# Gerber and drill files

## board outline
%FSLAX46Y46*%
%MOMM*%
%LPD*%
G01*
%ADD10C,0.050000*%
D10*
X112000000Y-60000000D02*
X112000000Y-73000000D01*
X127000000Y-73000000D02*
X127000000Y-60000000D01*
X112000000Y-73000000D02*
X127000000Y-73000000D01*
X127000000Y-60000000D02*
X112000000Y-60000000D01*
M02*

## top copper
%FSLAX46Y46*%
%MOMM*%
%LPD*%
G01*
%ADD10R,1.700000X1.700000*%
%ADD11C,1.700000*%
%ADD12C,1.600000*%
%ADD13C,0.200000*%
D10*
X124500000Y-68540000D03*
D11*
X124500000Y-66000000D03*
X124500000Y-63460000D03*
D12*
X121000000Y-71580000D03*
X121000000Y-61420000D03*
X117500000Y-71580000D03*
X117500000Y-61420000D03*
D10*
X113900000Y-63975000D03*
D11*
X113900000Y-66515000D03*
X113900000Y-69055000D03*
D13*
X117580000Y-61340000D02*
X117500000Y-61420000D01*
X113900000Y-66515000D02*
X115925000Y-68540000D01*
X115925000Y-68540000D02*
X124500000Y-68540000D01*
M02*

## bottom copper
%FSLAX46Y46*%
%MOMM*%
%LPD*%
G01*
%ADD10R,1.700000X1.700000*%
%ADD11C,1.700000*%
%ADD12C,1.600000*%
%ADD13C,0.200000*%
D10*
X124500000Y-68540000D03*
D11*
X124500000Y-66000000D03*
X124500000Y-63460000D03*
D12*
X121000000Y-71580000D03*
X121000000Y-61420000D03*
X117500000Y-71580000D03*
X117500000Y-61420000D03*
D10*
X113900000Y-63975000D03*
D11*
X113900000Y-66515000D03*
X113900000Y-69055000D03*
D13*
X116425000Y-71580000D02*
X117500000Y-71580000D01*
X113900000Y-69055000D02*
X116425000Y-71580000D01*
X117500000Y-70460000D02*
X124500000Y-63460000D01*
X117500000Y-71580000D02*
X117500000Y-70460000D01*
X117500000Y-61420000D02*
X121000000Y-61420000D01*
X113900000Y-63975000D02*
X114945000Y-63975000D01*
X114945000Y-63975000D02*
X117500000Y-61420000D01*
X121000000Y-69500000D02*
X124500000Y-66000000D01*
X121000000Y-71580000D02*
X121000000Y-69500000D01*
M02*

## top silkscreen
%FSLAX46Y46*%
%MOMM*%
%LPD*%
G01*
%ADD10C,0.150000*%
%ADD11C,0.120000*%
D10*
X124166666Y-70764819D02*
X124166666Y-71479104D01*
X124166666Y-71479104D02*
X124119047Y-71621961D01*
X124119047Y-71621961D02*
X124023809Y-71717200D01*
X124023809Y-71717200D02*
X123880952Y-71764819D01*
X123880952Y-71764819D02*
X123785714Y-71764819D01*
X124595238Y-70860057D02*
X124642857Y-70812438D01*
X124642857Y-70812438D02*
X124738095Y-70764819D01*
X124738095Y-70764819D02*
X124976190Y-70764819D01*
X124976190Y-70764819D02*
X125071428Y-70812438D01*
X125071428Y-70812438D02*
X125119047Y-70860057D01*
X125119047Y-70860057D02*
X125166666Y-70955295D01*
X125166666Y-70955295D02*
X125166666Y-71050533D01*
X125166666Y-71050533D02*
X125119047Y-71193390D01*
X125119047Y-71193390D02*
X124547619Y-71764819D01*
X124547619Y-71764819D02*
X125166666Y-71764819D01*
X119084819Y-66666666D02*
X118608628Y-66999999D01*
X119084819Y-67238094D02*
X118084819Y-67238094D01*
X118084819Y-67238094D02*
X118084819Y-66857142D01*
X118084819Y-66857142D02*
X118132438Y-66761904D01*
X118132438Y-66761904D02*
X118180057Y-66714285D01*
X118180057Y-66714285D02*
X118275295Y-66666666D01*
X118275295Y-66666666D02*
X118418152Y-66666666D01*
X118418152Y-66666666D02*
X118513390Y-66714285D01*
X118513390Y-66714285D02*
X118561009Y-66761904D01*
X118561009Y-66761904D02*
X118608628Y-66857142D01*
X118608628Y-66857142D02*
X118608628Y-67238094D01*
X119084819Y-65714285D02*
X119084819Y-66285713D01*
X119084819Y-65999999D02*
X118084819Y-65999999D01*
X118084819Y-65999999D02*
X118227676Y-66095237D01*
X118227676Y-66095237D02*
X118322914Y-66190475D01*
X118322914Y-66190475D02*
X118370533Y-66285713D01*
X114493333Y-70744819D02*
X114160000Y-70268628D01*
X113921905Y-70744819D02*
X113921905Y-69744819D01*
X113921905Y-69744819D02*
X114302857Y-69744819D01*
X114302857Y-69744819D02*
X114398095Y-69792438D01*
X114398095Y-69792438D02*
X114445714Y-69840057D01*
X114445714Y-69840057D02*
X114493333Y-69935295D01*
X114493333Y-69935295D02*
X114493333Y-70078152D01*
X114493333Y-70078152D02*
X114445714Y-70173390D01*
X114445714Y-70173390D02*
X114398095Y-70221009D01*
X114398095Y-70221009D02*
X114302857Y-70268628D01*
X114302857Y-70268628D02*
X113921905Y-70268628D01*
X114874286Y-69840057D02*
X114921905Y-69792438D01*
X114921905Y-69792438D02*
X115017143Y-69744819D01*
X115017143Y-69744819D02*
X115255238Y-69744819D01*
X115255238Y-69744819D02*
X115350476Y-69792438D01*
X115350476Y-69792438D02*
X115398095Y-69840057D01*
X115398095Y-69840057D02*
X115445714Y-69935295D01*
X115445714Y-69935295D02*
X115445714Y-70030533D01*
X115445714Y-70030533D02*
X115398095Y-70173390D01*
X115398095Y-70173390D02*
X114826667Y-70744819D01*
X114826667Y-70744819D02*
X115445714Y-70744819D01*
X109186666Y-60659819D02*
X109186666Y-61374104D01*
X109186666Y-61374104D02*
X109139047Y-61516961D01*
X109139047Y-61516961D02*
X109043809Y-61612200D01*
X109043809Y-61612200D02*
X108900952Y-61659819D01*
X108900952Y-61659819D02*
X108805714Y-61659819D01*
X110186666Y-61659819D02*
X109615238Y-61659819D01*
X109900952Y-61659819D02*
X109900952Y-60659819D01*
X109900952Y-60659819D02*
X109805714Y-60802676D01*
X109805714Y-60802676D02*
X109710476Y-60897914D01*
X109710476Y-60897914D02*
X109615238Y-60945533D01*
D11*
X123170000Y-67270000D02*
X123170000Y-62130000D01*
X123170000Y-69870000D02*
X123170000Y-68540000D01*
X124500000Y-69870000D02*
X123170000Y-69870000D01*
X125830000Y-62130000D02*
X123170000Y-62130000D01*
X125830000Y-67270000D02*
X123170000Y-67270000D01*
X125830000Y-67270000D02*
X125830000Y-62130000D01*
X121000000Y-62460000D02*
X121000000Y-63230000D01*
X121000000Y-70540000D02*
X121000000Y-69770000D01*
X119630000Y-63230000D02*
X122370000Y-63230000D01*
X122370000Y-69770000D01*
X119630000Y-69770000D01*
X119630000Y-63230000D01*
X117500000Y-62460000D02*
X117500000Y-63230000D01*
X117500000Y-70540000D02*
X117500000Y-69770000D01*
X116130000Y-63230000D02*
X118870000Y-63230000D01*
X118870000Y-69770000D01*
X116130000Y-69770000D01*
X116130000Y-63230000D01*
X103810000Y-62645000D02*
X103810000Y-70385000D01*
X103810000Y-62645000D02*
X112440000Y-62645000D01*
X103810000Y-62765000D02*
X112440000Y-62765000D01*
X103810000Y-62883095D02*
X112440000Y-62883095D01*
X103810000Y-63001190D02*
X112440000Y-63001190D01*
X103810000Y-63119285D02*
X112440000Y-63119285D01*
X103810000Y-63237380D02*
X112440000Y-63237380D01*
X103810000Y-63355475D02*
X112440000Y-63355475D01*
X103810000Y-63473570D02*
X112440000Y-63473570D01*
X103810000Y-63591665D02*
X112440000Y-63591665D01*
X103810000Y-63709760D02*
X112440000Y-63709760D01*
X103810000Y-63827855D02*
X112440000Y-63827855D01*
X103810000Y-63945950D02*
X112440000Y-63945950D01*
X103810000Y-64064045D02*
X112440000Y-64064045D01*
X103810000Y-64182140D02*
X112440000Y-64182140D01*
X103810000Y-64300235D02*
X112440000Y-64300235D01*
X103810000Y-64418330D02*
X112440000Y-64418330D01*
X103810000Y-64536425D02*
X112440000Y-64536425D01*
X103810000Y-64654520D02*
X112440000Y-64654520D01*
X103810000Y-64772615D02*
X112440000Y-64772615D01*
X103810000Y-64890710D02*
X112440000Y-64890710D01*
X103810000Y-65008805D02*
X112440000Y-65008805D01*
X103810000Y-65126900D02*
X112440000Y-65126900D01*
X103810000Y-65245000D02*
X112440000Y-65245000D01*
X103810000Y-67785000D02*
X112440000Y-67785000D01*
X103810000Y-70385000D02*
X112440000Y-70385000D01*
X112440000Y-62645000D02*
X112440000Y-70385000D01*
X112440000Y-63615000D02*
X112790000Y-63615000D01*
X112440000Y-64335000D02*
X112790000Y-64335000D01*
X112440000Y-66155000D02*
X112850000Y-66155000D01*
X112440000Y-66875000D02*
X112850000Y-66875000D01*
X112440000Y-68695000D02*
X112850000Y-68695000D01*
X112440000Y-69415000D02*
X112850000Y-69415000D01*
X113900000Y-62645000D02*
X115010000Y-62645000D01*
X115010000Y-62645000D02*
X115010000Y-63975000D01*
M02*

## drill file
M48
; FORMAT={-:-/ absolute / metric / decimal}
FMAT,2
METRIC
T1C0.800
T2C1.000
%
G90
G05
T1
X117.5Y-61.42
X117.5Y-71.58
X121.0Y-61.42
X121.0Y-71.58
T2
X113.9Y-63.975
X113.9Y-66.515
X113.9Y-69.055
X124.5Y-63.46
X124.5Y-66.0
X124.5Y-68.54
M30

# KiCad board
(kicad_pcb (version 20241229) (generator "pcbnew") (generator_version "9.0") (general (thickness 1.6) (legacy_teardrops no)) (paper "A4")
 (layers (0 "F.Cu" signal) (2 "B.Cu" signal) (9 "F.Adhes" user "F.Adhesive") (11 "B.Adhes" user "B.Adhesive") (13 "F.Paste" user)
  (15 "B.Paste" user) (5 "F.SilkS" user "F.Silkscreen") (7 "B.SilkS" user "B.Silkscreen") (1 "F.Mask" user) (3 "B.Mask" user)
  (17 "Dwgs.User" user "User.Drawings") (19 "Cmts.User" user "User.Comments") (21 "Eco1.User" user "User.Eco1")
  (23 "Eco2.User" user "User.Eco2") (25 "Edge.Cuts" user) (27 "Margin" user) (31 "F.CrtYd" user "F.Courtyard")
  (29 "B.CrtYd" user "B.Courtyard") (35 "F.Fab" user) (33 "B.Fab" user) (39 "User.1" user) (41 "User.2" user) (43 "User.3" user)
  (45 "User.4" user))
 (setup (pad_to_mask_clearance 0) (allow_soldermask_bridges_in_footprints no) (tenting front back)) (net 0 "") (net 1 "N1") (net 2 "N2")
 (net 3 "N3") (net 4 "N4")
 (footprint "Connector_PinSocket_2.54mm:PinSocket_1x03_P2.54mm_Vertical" (layer "F.Cu") (at 124.5 68.54 180)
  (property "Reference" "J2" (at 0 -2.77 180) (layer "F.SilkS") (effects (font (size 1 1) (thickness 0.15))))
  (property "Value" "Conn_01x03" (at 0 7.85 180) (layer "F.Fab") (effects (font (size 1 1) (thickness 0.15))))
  (fp_line (start 1.33 1.27) (end 1.33 6.41) (stroke (width 0.12) (type solid)) (layer "F.SilkS"))
  (fp_line (start 1.33 -1.33) (end 1.33 0) (stroke (width 0.12) (type solid)) (layer "F.SilkS"))
  (fp_line (start 0 -1.33) (end 1.33 -1.33) (stroke (width 0.12) (type solid)) (layer "F.SilkS"))
  (fp_line (start -1.33 6.41) (end 1.33 6.41) (stroke (width 0.12) (type solid)) (layer "F.SilkS"))
  (fp_line (start -1.33 1.27) (end 1.33 1.27) (stroke (width 0.12) (type solid)) (layer "F.SilkS"))
  (fp_line (start -1.33 1.27) (end -1.33 6.41) (stroke (width 0.12) (type solid)) (layer "F.SilkS"))
  (pad "1" thru_hole rect (at 0 0 180) (size 1.7 1.7) (drill 1) (layers "*.Cu" "*.Mask") (remove_unused_layers no) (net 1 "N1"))
  (pad "2" thru_hole circle (at 0 2.54 180) (size 1.7 1.7) (drill 1) (layers "*.Cu" "*.Mask") (remove_unused_layers no) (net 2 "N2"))
  (pad "3" thru_hole circle (at 0 5.08 180) (size 1.7 1.7) (drill 1) (layers "*.Cu" "*.Mask") (remove_unused_layers no) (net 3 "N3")))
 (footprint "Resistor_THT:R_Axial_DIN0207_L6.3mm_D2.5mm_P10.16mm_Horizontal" (layer "F.Cu") (at 121 71.58 90)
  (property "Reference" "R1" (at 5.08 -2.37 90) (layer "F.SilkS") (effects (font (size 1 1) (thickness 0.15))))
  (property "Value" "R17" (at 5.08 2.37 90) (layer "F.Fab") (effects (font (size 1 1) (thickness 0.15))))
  (fp_line (start 9.12 0) (end 8.35 0) (stroke (width 0.12) (type solid)) (layer "F.SilkS"))
  (fp_line (start 1.04 0) (end 1.81 0) (stroke (width 0.12) (type solid)) (layer "F.SilkS"))
  (fp_rect (start 1.81 -1.37) (end 8.35 1.37) (stroke (width 0.12) (type solid)) (fill no) (layer "F.SilkS"))
  (pad "1" thru_hole circle (at 0 0 90) (size 1.6 1.6) (drill 0.8) (layers "*.Cu" "*.Mask") (remove_unused_layers no) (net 2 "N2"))
  (pad "2" thru_hole circle (at 10.16 0 90) (size 1.6 1.6) (drill 0.8) (layers "*.Cu" "*.Mask") (remove_unused_layers no) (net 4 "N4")))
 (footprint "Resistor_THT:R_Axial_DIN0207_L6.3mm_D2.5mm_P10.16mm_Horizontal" (layer "F.Cu") (at 117.5 71.58 90)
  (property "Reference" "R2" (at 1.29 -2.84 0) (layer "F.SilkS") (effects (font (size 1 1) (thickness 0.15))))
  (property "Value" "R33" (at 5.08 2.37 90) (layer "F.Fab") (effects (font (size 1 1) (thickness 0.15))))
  (fp_line (start 9.12 0) (end 8.35 0) (stroke (width 0.12) (type solid)) (layer "F.SilkS"))
  (fp_line (start 1.04 0) (end 1.81 0) (stroke (width 0.12) (type solid)) (layer "F.SilkS"))
  (fp_rect (start 1.81 -1.37) (end 8.35 1.37) (stroke (width 0.12) (type solid)) (fill no) (layer "F.SilkS"))
  (pad "1" thru_hole circle (at 0 0 90) (size 1.6 1.6) (drill 0.8) (layers "*.Cu" "*.Mask") (remove_unused_layers no) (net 3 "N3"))
  (pad "2" thru_hole circle (at 10.16 0 90) (size 1.6 1.6) (drill 0.8) (layers "*.Cu" "*.Mask") (remove_unused_layers no) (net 4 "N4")))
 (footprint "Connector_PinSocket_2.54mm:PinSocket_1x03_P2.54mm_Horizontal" (layer "F.Cu") (at 113.9 63.975)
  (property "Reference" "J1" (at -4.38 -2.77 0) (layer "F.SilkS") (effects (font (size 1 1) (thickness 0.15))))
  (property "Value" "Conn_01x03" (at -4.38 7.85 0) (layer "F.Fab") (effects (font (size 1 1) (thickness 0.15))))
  (fp_line (start -10.09 -1.33) (end -10.09 6.41) (stroke (width 0.12) (type solid)) (layer "F.SilkS"))
  (fp_line (start -10.09 -1.33) (end -1.46 -1.33) (stroke (width 0.12) (type solid)) (layer "F.SilkS"))
  (fp_line (start -10.09 -1.21) (end -1.46 -1.21) (stroke (width 0.12) (type solid)) (layer "F.SilkS"))
  (fp_line (start -10.09 -1.091905) (end -1.46 -1.091905) (stroke (width 0.12) (type solid)) (layer "F.SilkS"))
  (fp_line (start -10.09 -0.97381) (end -1.46 -0.97381) (stroke (width 0.12) (type solid)) (layer "F.SilkS"))
  (fp_line (start -10.09 -0.855715) (end -1.46 -0.855715) (stroke (width 0.12) (type solid)) (layer "F.SilkS"))
  (fp_line (start -10.09 -0.73762) (end -1.46 -0.73762) (stroke (width 0.12) (type solid)) (layer "F.SilkS"))
  (fp_line (start -10.09 -0.619525) (end -1.46 -0.619525) (stroke (width 0.12) (type solid)) (layer "F.SilkS"))
  (fp_line (start -10.09 -0.50143) (end -1.46 -0.50143) (stroke (width 0.12) (type solid)) (layer "F.SilkS"))
  (fp_line (start -10.09 -0.383335) (end -1.46 -0.383335) (stroke (width 0.12) (type solid)) (layer "F.SilkS"))
  (fp_line (start -10.09 -0.26524) (end -1.46 -0.26524) (stroke (width 0.12) (type solid)) (layer "F.SilkS"))
  (fp_line (start -10.09 -0.147145) (end -1.46 -0.147145) (stroke (width 0.12) (type solid)) (layer "F.SilkS"))
  (fp_line (start -10.09 -0.02905) (end -1.46 -0.02905) (stroke (width 0.12) (type solid)) (layer "F.SilkS"))
  (fp_line (start -10.09 0.089045) (end -1.46 0.089045) (stroke (width 0.12) (type solid)) (layer "F.SilkS"))
  (fp_line (start -10.09 0.20714) (end -1.46 0.20714) (stroke (width 0.12) (type solid)) (layer "F.SilkS"))
  (fp_line (start -10.09 0.325235) (end -1.46 0.325235) (stroke (width 0.12) (type solid)) (layer "F.SilkS"))
  (fp_line (start -10.09 0.44333) (end -1.46 0.44333) (stroke (width 0.12) (type solid)) (layer "F.SilkS"))
  (fp_line (start -10.09 0.561425) (end -1.46 0.561425) (stroke (width 0.12) (type solid)) (layer "F.SilkS"))
  (fp_line (start -10.09 0.67952) (end -1.46 0.67952) (stroke (width 0.12) (type solid)) (layer "F.SilkS"))
  (fp_line (start -10.09 0.797615) (end -1.46 0.797615) (stroke (width 0.12) (type solid)) (layer "F.SilkS"))
  (fp_line (start -10.09 0.91571) (end -1.46 0.91571) (stroke (width 0.12) (type solid)) (layer "F.SilkS"))
  (fp_line (start -10.09 1.033805) (end -1.46 1.033805) (stroke (width 0.12) (type solid)) (layer "F.SilkS"))
  (fp_line (start -10.09 1.1519) (end -1.46 1.1519) (stroke (width 0.12) (type solid)) (layer "F.SilkS"))
  (fp_line (start -10.09 1.27) (end -1.46 1.27) (stroke (width 0.12) (type solid)) (layer "F.SilkS"))
  (fp_line (start -10.09 3.81) (end -1.46 3.81) (stroke (width 0.12) (type solid)) (layer "F.SilkS"))
  (fp_line (start -10.09 6.41) (end -1.46 6.41) (stroke (width 0.12) (type solid)) (layer "F.SilkS"))
  (fp_line (start -1.46 -1.33) (end -1.46 6.41) (stroke (width 0.12) (type solid)) (layer "F.SilkS"))
  (fp_line (start -1.46 -0.36) (end -1.11 -0.36) (stroke (width 0.12) (type solid)) (layer "F.SilkS"))
  (fp_line (start -1.46 0.36) (end -1.11 0.36) (stroke (width 0.12) (type solid)) (layer "F.SilkS"))
  (fp_line (start -1.46 2.18) (end -1.05 2.18) (stroke (width 0.12) (type solid)) (layer "F.SilkS"))
  (fp_line (start -1.46 2.9) (end -1.05 2.9) (stroke (width 0.12) (type solid)) (layer "F.SilkS"))
  (fp_line (start -1.46 4.72) (end -1.05 4.72) (stroke (width 0.12) (type solid)) (layer "F.SilkS"))
  (fp_line (start -1.46 5.44) (end -1.05 5.44) (stroke (width 0.12) (type solid)) (layer "F.SilkS"))
  (fp_line (start 0 -1.33) (end 1.11 -1.33) (stroke (width 0.12) (type solid)) (layer "F.SilkS"))
  (fp_line (start 1.11 -1.33) (end 1.11 0) (stroke (width 0.12) (type solid)) (layer "F.SilkS"))
  (pad "1" thru_hole rect (at 0 0) (size 1.7 1.7) (drill 1) (layers "*.Cu" "*.Mask") (remove_unused_layers no) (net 4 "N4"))
  (pad "2" thru_hole circle (at 0 2.54) (size 1.7 1.7) (drill 1) (layers "*.Cu" "*.Mask") (remove_unused_layers no) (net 1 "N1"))
  (pad "3" thru_hole circle (at 0 5.08) (size 1.7 1.7) (drill 1) (layers "*.Cu" "*.Mask") (remove_unused_layers no) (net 3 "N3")))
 (gr_line (start 112 60) (end 112 73) (stroke (width 0.05) (type default)) (layer "Edge.Cuts"))
 (gr_line (start 127 73) (end 127 60) (stroke (width 0.05) (type default)) (layer "Edge.Cuts"))
 (gr_line (start 112 73) (end 127 73) (stroke (width 0.05) (type default)) (layer "Edge.Cuts"))
 (gr_line (start 127 60) (end 112 60) (stroke (width 0.05) (type default)) (layer "Edge.Cuts"))
 (segment (start 116.425 71.58) (end 117.5 71.58) (width 0.2) (layer "B.Cu") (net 3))
 (segment (start 113.9 69.055) (end 116.425 71.58) (width 0.2) (layer "B.Cu") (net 3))
 (segment (start 117.5 70.46) (end 124.5 63.46) (width 0.2) (layer "B.Cu") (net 3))
 (segment (start 117.5 71.58) (end 117.5 70.46) (width 0.2) (layer "B.Cu") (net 3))
 (segment (start 117.58 61.34) (end 117.5 61.42) (width 0.2) (layer "F.Cu") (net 4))
 (segment (start 117.5 61.42) (end 121 61.42) (width 0.2) (layer "B.Cu") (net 4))
 (segment (start 113.9 63.975) (end 114.945 63.975) (width 0.2) (layer "B.Cu") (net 4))
 (segment (start 114.945 63.975) (end 117.5 61.42) (width 0.2) (layer "B.Cu") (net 4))
 (segment (start 113.9 66.515) (end 115.925 68.54) (width 0.2) (layer "F.Cu") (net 1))
 (segment (start 115.925 68.54) (end 124.5 68.54) (width 0.2) (layer "F.Cu") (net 1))
 (segment (start 121 69.5) (end 124.5 66) (width 0.2) (layer "B.Cu") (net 2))
 (segment (start 121 71.58) (end 121 69.5) (width 0.2) (layer "B.Cu") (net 2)))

